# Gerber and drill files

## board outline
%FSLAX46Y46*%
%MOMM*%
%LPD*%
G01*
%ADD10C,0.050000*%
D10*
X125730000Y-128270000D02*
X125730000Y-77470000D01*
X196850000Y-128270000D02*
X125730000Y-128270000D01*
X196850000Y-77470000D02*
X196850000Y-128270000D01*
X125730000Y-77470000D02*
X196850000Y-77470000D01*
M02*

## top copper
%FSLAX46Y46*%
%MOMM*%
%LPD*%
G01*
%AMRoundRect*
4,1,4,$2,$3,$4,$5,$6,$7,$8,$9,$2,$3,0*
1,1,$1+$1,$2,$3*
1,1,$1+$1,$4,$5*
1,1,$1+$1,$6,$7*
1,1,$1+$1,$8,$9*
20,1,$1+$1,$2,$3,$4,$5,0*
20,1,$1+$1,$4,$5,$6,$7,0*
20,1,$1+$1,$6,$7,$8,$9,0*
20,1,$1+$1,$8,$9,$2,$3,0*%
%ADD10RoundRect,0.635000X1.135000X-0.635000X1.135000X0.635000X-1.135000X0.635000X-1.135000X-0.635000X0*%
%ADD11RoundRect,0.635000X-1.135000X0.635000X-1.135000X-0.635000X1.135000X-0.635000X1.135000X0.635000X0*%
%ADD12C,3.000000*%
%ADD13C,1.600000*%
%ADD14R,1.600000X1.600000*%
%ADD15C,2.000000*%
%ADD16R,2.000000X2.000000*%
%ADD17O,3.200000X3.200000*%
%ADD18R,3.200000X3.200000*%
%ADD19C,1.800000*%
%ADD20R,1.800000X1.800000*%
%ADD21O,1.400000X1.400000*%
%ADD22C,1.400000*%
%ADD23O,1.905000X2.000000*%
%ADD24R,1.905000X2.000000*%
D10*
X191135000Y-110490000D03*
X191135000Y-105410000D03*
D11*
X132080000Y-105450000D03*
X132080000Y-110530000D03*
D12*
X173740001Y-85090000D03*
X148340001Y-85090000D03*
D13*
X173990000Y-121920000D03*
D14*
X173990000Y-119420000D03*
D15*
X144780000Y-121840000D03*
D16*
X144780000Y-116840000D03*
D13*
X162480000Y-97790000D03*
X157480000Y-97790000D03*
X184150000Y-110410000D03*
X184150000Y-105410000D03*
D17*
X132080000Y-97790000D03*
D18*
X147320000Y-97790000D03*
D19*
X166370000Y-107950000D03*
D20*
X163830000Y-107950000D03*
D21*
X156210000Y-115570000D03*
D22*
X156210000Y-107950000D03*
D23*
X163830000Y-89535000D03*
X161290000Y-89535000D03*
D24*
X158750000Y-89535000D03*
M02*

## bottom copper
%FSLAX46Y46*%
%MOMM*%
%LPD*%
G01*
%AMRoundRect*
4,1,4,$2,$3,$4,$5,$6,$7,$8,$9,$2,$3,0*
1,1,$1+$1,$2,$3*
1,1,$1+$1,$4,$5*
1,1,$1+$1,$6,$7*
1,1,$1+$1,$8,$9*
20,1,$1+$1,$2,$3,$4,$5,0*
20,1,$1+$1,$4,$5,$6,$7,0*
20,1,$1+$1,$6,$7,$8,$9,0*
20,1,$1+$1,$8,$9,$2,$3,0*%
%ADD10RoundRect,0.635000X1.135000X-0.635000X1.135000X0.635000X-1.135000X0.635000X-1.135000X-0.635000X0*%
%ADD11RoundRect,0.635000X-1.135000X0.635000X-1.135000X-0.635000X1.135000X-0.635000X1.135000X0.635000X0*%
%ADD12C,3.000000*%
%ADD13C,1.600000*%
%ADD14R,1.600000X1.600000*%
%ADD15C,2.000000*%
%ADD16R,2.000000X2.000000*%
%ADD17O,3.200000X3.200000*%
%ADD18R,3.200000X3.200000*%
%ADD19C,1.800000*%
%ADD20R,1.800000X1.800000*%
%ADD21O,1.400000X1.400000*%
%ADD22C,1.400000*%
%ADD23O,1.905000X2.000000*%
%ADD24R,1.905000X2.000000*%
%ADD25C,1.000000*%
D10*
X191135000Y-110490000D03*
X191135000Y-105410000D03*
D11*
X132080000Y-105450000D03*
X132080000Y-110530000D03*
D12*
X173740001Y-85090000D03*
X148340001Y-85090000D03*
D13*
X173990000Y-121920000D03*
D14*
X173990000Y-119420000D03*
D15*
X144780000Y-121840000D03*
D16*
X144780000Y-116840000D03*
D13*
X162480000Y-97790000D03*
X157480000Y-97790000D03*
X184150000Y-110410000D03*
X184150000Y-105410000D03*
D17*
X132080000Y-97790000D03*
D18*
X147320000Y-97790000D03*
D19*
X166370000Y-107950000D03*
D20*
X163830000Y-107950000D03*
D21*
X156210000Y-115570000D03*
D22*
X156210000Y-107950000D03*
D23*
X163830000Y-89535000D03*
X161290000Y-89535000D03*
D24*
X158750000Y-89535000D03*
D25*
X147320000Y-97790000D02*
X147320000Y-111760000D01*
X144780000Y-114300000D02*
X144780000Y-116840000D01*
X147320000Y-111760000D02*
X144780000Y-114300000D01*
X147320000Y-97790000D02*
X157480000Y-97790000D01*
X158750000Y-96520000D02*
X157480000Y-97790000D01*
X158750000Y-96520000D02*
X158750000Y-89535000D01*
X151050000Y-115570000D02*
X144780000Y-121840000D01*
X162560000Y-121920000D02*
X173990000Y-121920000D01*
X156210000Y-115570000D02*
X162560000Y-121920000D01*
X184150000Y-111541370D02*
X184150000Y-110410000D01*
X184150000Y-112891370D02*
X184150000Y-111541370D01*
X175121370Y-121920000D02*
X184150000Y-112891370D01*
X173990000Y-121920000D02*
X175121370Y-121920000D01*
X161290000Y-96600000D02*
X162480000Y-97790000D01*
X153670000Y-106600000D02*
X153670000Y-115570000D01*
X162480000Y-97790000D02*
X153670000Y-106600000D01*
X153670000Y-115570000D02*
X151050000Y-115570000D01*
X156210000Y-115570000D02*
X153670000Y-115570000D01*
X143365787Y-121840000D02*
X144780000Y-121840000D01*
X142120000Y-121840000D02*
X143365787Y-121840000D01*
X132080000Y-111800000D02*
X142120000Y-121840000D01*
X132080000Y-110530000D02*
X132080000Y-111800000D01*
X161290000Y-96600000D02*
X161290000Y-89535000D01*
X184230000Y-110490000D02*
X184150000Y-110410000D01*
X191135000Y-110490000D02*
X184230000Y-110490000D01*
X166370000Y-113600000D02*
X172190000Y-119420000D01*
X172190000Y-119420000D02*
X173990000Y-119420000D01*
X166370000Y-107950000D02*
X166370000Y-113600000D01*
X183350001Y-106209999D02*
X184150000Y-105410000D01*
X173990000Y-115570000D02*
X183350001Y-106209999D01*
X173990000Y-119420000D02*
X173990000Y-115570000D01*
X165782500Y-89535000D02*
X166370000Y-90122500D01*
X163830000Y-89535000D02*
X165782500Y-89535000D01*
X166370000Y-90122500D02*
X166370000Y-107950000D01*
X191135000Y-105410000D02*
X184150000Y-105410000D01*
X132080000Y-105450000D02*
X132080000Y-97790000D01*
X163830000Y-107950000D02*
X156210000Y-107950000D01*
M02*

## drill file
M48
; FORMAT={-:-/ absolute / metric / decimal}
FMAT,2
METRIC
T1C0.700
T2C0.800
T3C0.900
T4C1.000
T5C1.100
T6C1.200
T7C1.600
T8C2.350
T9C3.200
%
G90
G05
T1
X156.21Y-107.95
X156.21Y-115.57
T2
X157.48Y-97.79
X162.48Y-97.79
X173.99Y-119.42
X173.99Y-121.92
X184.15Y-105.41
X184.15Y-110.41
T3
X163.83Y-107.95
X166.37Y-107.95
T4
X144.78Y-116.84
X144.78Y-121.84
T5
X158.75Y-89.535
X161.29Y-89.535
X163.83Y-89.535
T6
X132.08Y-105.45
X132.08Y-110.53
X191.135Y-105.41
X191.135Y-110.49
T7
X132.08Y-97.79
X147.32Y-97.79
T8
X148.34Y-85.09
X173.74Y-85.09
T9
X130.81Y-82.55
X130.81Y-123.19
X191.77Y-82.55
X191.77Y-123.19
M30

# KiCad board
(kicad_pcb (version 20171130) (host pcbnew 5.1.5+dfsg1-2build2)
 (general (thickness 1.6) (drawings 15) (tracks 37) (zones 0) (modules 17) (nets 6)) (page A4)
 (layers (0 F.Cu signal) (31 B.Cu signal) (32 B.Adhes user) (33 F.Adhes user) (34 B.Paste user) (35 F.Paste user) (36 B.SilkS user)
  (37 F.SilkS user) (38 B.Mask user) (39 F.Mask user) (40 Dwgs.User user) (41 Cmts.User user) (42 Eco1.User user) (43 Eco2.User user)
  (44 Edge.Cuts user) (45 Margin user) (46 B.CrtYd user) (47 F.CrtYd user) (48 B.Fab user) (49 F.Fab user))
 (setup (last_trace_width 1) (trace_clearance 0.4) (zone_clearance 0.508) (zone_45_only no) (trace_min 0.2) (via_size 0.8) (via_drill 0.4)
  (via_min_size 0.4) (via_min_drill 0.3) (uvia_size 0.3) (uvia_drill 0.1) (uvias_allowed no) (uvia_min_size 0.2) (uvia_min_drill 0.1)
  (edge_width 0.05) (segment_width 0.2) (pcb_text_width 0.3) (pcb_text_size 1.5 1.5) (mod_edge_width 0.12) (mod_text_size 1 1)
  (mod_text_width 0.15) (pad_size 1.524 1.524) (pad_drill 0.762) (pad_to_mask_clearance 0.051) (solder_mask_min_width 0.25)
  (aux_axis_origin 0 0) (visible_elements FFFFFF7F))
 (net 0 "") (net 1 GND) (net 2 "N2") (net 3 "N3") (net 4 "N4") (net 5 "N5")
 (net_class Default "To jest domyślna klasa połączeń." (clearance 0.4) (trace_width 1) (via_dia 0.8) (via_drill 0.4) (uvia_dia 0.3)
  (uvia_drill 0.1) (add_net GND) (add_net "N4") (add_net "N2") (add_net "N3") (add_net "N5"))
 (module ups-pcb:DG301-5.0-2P (layer F.Cu) (at 191.135 107.99 90)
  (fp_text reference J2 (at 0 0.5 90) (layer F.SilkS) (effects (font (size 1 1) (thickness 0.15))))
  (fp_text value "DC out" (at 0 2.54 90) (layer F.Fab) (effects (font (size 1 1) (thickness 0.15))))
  (pad 1 thru_hole roundrect (at -2.5 0 90) (size 2.54 3.54) (drill 1.2) (layers *.Cu *.Mask) (roundrect_rratio 0.25) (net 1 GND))
  (pad 2 thru_hole roundrect (at 2.58 0 90) (size 2.54 3.54) (drill 1.2) (layers *.Cu *.Mask) (roundrect_rratio 0.25) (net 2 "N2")))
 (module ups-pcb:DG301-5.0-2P (layer F.Cu) (at 132.08 107.95 270)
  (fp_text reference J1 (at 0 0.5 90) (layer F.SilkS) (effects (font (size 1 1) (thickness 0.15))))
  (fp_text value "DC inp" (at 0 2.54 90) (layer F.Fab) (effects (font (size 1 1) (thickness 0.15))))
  (pad 1 thru_hole roundrect (at -2.5 0 270) (size 2.54 3.54) (drill 1.2) (layers *.Cu *.Mask) (roundrect_rratio 0.25) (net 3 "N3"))
  (pad 2 thru_hole roundrect (at 2.58 0 270) (size 2.54 3.54) (drill 1.2) (layers *.Cu *.Mask) (roundrect_rratio 0.25) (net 1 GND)))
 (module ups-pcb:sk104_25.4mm (layer F.Cu) (at 161.040001 85.09)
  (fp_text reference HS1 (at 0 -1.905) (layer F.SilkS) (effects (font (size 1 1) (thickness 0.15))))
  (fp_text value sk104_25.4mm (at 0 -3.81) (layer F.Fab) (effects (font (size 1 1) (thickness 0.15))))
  (pad "" np_thru_hole circle (at 12.7 0) (size 3 3) (drill 2.35) (layers *.Cu *.Mask))
  (pad "" np_thru_hole circle (at -12.7 0) (size 3 3) (drill 2.35) (layers *.Cu *.Mask)))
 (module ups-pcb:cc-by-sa (layer F.Cu) (at 159.385 121.92)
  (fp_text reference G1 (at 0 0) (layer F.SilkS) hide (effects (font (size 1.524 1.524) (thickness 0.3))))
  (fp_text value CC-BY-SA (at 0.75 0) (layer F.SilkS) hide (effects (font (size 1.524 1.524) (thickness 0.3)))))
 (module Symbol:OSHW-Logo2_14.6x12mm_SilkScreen (layer F.Cu) (at 186.055 93.98)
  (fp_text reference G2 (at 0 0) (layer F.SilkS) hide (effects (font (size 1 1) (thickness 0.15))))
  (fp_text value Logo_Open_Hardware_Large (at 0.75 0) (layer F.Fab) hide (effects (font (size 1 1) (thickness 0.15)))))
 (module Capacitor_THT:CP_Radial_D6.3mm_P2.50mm (layer F.Cu) (at 173.99 119.42 270)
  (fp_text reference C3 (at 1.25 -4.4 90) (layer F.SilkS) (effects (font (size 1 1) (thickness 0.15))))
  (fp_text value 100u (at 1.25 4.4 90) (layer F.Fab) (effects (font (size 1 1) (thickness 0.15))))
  (pad 2 thru_hole circle (at 2.5 0 270) (size 1.6 1.6) (drill 0.8) (layers *.Cu *.Mask) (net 1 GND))
  (pad 1 thru_hole rect (at 0 0 270) (size 1.6 1.6) (drill 0.8) (layers *.Cu *.Mask) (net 2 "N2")))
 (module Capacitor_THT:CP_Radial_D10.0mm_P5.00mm (layer F.Cu) (at 144.78 116.84 270)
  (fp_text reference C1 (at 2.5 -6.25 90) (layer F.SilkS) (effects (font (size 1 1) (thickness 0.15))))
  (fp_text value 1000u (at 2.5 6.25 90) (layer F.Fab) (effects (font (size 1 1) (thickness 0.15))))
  (pad 2 thru_hole circle (at 5 0 270) (size 2 2) (drill 1) (layers *.Cu *.Mask) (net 1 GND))
  (pad 1 thru_hole rect (at 0 0 270) (size 2 2) (drill 1) (layers *.Cu *.Mask) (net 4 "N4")))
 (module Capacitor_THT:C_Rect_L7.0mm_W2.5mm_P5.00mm (layer F.Cu) (at 157.48 97.79)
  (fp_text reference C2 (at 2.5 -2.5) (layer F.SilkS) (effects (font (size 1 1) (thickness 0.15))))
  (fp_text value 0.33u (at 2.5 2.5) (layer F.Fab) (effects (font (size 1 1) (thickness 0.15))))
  (pad 2 thru_hole circle (at 5 0) (size 1.6 1.6) (drill 0.8) (layers *.Cu *.Mask) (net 1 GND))
  (pad 1 thru_hole circle (at 0 0) (size 1.6 1.6) (drill 0.8) (layers *.Cu *.Mask) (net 4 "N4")))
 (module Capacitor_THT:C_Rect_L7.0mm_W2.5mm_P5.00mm (layer F.Cu) (at 184.15 105.41 270)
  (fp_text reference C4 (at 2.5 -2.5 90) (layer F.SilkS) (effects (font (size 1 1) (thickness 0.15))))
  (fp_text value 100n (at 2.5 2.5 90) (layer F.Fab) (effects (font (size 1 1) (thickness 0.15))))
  (pad 2 thru_hole circle (at 5 0 270) (size 1.6 1.6) (drill 0.8) (layers *.Cu *.Mask) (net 1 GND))
  (pad 1 thru_hole circle (at 0 0 270) (size 1.6 1.6) (drill 0.8) (layers *.Cu *.Mask) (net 2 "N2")))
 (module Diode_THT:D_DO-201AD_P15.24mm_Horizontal (layer F.Cu) (at 147.32 97.79 180)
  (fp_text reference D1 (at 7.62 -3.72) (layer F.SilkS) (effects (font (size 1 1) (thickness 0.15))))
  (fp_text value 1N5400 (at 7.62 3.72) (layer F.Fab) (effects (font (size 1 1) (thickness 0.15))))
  (pad 2 thru_hole oval (at 15.24 0 180) (size 3.2 3.2) (drill 1.6) (layers *.Cu *.Mask) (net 3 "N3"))
  (pad 1 thru_hole rect (at 0 0 180) (size 3.2 3.2) (drill 1.6) (layers *.Cu *.Mask) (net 4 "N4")))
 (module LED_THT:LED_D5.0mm (layer F.Cu) (at 163.83 107.95)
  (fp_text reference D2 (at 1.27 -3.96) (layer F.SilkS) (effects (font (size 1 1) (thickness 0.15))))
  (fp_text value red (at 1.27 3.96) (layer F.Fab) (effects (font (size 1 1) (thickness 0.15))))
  (pad 2 thru_hole circle (at 2.54 0) (size 1.8 1.8) (drill 0.9) (layers *.Cu *.Mask) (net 2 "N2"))
  (pad 1 thru_hole rect (at 0 0) (size 1.8 1.8) (drill 0.9) (layers *.Cu *.Mask) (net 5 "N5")))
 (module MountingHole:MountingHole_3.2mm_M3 (layer F.Cu) (at 130.81 82.55)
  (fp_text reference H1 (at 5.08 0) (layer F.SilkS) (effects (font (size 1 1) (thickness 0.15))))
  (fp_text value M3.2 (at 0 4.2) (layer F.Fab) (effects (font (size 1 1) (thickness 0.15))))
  (pad 1 np_thru_hole circle (at 0 0) (size 3.2 3.2) (drill 3.2) (layers *.Cu *.Mask)))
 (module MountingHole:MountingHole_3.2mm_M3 (layer F.Cu) (at 191.77 82.55)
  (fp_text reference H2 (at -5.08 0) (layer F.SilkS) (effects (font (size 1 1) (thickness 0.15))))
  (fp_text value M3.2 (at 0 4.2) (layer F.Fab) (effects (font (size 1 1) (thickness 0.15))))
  (pad 1 np_thru_hole circle (at 0 0) (size 3.2 3.2) (drill 3.2) (layers *.Cu *.Mask)))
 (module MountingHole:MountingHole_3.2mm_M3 (layer F.Cu) (at 191.77 123.19)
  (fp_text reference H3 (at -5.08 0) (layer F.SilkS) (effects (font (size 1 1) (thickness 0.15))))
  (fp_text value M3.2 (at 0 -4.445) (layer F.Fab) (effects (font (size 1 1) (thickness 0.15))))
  (pad 1 np_thru_hole circle (at 0 0) (size 3.2 3.2) (drill 3.2) (layers *.Cu *.Mask)))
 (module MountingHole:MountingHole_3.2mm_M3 (layer F.Cu) (at 130.81 123.19)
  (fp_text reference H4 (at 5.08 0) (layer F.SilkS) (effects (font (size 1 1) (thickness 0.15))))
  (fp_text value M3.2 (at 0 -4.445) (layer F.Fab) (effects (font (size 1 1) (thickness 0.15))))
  (pad 1 np_thru_hole circle (at 0 0) (size 3.2 3.2) (drill 3.2) (layers *.Cu *.Mask)))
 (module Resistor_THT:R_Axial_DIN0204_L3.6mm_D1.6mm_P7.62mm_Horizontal (layer F.Cu) (at 156.21 107.95 270)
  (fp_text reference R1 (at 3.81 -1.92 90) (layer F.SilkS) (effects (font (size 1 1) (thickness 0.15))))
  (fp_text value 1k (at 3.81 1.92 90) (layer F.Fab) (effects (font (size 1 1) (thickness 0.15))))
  (pad 2 thru_hole oval (at 7.62 0 270) (size 1.4 1.4) (drill 0.7) (layers *.Cu *.Mask) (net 1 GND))
  (pad 1 thru_hole circle (at 0 0 270) (size 1.4 1.4) (drill 0.7) (layers *.Cu *.Mask) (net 5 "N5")))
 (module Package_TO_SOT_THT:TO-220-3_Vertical (layer F.Cu) (at 158.75 89.535)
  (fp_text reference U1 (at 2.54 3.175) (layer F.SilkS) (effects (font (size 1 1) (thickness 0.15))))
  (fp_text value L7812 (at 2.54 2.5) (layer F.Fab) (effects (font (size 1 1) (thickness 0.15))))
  (pad 3 thru_hole oval (at 5.08 0) (size 1.905 2) (drill 1.1) (layers *.Cu *.Mask) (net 2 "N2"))
  (pad 2 thru_hole oval (at 2.54 0) (size 1.905 2) (drill 1.1) (layers *.Cu *.Mask) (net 1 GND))
  (pad 1 thru_hole rect (at 0 0) (size 1.905 2) (drill 1.1) (layers *.Cu *.Mask) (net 4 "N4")))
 (gr_line (start 125.73 128.27) (end 125.73 77.47) (layer Edge.Cuts) (width 0.05))
 (gr_line (start 196.85 128.27) (end 125.73 128.27) (layer Edge.Cuts) (width 0.05))
 (gr_line (start 196.85 77.47) (end 196.85 128.27) (layer Edge.Cuts) (width 0.05))
 (gr_line (start 125.73 77.47) (end 196.85 77.47) (layer Edge.Cuts) (width 0.05))
 (segment (start 147.32 97.79) (end 147.32 111.76) (width 1) (layer B.Cu) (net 4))
 (segment (start 144.78 114.3) (end 144.78 116.84) (width 1) (layer B.Cu) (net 4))
 (segment (start 147.32 111.76) (end 144.78 114.3) (width 1) (layer B.Cu) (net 4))
 (segment (start 147.32 97.79) (end 157.48 97.79) (width 1) (layer B.Cu) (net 4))
 (segment (start 158.75 96.52) (end 157.48 97.79) (width 1) (layer B.Cu) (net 4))
 (segment (start 158.75 96.52) (end 158.75 89.535) (width 1) (layer B.Cu) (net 4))
 (segment (start 151.05 115.57) (end 144.78 121.84) (width 1) (layer B.Cu) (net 1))
 (segment (start 162.56 121.92) (end 173.99 121.92) (width 1) (layer B.Cu) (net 1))
 (segment (start 156.21 115.57) (end 162.56 121.92) (width 1) (layer B.Cu) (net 1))
 (segment (start 184.15 111.54137) (end 184.15 110.41) (width 1) (layer B.Cu) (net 1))
 (segment (start 184.15 112.89137) (end 184.15 111.54137) (width 1) (layer B.Cu) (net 1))
 (segment (start 175.12137 121.92) (end 184.15 112.89137) (width 1) (layer B.Cu) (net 1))
 (segment (start 173.99 121.92) (end 175.12137 121.92) (width 1) (layer B.Cu) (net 1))
 (segment (start 161.29 96.6) (end 162.48 97.79) (width 1) (layer B.Cu) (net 1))
 (segment (start 153.67 106.6) (end 153.67 115.57) (width 1) (layer B.Cu) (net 1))
 (segment (start 162.48 97.79) (end 153.67 106.6) (width 1) (layer B.Cu) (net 1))
 (segment (start 153.67 115.57) (end 151.05 115.57) (width 1) (layer B.Cu) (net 1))
 (segment (start 156.21 115.57) (end 153.67 115.57) (width 1) (layer B.Cu) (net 1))
 (segment (start 143.365787 121.84) (end 144.78 121.84) (width 1) (layer B.Cu) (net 1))
 (segment (start 142.12 121.84) (end 143.365787 121.84) (width 1) (layer B.Cu) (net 1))
 (segment (start 132.08 111.8) (end 142.12 121.84) (width 1) (layer B.Cu) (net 1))
 (segment (start 132.08 110.53) (end 132.08 111.8) (width 1) (layer B.Cu) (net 1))
 (segment (start 161.29 96.6) (end 161.29 89.535) (width 1) (layer B.Cu) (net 1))
 (segment (start 184.23 110.49) (end 184.15 110.41) (width 1) (layer B.Cu) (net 1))
 (segment (start 191.135 110.49) (end 184.23 110.49) (width 1) (layer B.Cu) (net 1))
 (segment (start 166.37 113.6) (end 172.19 119.42) (width 1) (layer B.Cu) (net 2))
 (segment (start 172.19 119.42) (end 173.99 119.42) (width 1) (layer B.Cu) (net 2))
 (segment (start 166.37 107.95) (end 166.37 113.6) (width 1) (layer B.Cu) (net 2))
 (segment (start 183.350001 106.209999) (end 184.15 105.41) (width 1) (layer B.Cu) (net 2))
 (segment (start 173.99 115.57) (end 183.350001 106.209999) (width 1) (layer B.Cu) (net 2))
 (segment (start 173.99 119.42) (end 173.99 115.57) (width 1) (layer B.Cu) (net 2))
 (segment (start 165.7825 89.535) (end 166.37 90.1225) (width 1) (layer B.Cu) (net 2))
 (segment (start 163.83 89.535) (end 165.7825 89.535) (width 1) (layer B.Cu) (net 2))
 (segment (start 166.37 90.1225) (end 166.37 107.95) (width 1) (layer B.Cu) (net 2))
 (segment (start 191.135 105.41) (end 184.15 105.41) (width 1) (layer B.Cu) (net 2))
 (segment (start 132.08 105.45) (end 132.08 97.79) (width 1) (layer B.Cu) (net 3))
 (segment (start 163.83 107.95) (end 156.21 107.95) (width 1) (layer B.Cu) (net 5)))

